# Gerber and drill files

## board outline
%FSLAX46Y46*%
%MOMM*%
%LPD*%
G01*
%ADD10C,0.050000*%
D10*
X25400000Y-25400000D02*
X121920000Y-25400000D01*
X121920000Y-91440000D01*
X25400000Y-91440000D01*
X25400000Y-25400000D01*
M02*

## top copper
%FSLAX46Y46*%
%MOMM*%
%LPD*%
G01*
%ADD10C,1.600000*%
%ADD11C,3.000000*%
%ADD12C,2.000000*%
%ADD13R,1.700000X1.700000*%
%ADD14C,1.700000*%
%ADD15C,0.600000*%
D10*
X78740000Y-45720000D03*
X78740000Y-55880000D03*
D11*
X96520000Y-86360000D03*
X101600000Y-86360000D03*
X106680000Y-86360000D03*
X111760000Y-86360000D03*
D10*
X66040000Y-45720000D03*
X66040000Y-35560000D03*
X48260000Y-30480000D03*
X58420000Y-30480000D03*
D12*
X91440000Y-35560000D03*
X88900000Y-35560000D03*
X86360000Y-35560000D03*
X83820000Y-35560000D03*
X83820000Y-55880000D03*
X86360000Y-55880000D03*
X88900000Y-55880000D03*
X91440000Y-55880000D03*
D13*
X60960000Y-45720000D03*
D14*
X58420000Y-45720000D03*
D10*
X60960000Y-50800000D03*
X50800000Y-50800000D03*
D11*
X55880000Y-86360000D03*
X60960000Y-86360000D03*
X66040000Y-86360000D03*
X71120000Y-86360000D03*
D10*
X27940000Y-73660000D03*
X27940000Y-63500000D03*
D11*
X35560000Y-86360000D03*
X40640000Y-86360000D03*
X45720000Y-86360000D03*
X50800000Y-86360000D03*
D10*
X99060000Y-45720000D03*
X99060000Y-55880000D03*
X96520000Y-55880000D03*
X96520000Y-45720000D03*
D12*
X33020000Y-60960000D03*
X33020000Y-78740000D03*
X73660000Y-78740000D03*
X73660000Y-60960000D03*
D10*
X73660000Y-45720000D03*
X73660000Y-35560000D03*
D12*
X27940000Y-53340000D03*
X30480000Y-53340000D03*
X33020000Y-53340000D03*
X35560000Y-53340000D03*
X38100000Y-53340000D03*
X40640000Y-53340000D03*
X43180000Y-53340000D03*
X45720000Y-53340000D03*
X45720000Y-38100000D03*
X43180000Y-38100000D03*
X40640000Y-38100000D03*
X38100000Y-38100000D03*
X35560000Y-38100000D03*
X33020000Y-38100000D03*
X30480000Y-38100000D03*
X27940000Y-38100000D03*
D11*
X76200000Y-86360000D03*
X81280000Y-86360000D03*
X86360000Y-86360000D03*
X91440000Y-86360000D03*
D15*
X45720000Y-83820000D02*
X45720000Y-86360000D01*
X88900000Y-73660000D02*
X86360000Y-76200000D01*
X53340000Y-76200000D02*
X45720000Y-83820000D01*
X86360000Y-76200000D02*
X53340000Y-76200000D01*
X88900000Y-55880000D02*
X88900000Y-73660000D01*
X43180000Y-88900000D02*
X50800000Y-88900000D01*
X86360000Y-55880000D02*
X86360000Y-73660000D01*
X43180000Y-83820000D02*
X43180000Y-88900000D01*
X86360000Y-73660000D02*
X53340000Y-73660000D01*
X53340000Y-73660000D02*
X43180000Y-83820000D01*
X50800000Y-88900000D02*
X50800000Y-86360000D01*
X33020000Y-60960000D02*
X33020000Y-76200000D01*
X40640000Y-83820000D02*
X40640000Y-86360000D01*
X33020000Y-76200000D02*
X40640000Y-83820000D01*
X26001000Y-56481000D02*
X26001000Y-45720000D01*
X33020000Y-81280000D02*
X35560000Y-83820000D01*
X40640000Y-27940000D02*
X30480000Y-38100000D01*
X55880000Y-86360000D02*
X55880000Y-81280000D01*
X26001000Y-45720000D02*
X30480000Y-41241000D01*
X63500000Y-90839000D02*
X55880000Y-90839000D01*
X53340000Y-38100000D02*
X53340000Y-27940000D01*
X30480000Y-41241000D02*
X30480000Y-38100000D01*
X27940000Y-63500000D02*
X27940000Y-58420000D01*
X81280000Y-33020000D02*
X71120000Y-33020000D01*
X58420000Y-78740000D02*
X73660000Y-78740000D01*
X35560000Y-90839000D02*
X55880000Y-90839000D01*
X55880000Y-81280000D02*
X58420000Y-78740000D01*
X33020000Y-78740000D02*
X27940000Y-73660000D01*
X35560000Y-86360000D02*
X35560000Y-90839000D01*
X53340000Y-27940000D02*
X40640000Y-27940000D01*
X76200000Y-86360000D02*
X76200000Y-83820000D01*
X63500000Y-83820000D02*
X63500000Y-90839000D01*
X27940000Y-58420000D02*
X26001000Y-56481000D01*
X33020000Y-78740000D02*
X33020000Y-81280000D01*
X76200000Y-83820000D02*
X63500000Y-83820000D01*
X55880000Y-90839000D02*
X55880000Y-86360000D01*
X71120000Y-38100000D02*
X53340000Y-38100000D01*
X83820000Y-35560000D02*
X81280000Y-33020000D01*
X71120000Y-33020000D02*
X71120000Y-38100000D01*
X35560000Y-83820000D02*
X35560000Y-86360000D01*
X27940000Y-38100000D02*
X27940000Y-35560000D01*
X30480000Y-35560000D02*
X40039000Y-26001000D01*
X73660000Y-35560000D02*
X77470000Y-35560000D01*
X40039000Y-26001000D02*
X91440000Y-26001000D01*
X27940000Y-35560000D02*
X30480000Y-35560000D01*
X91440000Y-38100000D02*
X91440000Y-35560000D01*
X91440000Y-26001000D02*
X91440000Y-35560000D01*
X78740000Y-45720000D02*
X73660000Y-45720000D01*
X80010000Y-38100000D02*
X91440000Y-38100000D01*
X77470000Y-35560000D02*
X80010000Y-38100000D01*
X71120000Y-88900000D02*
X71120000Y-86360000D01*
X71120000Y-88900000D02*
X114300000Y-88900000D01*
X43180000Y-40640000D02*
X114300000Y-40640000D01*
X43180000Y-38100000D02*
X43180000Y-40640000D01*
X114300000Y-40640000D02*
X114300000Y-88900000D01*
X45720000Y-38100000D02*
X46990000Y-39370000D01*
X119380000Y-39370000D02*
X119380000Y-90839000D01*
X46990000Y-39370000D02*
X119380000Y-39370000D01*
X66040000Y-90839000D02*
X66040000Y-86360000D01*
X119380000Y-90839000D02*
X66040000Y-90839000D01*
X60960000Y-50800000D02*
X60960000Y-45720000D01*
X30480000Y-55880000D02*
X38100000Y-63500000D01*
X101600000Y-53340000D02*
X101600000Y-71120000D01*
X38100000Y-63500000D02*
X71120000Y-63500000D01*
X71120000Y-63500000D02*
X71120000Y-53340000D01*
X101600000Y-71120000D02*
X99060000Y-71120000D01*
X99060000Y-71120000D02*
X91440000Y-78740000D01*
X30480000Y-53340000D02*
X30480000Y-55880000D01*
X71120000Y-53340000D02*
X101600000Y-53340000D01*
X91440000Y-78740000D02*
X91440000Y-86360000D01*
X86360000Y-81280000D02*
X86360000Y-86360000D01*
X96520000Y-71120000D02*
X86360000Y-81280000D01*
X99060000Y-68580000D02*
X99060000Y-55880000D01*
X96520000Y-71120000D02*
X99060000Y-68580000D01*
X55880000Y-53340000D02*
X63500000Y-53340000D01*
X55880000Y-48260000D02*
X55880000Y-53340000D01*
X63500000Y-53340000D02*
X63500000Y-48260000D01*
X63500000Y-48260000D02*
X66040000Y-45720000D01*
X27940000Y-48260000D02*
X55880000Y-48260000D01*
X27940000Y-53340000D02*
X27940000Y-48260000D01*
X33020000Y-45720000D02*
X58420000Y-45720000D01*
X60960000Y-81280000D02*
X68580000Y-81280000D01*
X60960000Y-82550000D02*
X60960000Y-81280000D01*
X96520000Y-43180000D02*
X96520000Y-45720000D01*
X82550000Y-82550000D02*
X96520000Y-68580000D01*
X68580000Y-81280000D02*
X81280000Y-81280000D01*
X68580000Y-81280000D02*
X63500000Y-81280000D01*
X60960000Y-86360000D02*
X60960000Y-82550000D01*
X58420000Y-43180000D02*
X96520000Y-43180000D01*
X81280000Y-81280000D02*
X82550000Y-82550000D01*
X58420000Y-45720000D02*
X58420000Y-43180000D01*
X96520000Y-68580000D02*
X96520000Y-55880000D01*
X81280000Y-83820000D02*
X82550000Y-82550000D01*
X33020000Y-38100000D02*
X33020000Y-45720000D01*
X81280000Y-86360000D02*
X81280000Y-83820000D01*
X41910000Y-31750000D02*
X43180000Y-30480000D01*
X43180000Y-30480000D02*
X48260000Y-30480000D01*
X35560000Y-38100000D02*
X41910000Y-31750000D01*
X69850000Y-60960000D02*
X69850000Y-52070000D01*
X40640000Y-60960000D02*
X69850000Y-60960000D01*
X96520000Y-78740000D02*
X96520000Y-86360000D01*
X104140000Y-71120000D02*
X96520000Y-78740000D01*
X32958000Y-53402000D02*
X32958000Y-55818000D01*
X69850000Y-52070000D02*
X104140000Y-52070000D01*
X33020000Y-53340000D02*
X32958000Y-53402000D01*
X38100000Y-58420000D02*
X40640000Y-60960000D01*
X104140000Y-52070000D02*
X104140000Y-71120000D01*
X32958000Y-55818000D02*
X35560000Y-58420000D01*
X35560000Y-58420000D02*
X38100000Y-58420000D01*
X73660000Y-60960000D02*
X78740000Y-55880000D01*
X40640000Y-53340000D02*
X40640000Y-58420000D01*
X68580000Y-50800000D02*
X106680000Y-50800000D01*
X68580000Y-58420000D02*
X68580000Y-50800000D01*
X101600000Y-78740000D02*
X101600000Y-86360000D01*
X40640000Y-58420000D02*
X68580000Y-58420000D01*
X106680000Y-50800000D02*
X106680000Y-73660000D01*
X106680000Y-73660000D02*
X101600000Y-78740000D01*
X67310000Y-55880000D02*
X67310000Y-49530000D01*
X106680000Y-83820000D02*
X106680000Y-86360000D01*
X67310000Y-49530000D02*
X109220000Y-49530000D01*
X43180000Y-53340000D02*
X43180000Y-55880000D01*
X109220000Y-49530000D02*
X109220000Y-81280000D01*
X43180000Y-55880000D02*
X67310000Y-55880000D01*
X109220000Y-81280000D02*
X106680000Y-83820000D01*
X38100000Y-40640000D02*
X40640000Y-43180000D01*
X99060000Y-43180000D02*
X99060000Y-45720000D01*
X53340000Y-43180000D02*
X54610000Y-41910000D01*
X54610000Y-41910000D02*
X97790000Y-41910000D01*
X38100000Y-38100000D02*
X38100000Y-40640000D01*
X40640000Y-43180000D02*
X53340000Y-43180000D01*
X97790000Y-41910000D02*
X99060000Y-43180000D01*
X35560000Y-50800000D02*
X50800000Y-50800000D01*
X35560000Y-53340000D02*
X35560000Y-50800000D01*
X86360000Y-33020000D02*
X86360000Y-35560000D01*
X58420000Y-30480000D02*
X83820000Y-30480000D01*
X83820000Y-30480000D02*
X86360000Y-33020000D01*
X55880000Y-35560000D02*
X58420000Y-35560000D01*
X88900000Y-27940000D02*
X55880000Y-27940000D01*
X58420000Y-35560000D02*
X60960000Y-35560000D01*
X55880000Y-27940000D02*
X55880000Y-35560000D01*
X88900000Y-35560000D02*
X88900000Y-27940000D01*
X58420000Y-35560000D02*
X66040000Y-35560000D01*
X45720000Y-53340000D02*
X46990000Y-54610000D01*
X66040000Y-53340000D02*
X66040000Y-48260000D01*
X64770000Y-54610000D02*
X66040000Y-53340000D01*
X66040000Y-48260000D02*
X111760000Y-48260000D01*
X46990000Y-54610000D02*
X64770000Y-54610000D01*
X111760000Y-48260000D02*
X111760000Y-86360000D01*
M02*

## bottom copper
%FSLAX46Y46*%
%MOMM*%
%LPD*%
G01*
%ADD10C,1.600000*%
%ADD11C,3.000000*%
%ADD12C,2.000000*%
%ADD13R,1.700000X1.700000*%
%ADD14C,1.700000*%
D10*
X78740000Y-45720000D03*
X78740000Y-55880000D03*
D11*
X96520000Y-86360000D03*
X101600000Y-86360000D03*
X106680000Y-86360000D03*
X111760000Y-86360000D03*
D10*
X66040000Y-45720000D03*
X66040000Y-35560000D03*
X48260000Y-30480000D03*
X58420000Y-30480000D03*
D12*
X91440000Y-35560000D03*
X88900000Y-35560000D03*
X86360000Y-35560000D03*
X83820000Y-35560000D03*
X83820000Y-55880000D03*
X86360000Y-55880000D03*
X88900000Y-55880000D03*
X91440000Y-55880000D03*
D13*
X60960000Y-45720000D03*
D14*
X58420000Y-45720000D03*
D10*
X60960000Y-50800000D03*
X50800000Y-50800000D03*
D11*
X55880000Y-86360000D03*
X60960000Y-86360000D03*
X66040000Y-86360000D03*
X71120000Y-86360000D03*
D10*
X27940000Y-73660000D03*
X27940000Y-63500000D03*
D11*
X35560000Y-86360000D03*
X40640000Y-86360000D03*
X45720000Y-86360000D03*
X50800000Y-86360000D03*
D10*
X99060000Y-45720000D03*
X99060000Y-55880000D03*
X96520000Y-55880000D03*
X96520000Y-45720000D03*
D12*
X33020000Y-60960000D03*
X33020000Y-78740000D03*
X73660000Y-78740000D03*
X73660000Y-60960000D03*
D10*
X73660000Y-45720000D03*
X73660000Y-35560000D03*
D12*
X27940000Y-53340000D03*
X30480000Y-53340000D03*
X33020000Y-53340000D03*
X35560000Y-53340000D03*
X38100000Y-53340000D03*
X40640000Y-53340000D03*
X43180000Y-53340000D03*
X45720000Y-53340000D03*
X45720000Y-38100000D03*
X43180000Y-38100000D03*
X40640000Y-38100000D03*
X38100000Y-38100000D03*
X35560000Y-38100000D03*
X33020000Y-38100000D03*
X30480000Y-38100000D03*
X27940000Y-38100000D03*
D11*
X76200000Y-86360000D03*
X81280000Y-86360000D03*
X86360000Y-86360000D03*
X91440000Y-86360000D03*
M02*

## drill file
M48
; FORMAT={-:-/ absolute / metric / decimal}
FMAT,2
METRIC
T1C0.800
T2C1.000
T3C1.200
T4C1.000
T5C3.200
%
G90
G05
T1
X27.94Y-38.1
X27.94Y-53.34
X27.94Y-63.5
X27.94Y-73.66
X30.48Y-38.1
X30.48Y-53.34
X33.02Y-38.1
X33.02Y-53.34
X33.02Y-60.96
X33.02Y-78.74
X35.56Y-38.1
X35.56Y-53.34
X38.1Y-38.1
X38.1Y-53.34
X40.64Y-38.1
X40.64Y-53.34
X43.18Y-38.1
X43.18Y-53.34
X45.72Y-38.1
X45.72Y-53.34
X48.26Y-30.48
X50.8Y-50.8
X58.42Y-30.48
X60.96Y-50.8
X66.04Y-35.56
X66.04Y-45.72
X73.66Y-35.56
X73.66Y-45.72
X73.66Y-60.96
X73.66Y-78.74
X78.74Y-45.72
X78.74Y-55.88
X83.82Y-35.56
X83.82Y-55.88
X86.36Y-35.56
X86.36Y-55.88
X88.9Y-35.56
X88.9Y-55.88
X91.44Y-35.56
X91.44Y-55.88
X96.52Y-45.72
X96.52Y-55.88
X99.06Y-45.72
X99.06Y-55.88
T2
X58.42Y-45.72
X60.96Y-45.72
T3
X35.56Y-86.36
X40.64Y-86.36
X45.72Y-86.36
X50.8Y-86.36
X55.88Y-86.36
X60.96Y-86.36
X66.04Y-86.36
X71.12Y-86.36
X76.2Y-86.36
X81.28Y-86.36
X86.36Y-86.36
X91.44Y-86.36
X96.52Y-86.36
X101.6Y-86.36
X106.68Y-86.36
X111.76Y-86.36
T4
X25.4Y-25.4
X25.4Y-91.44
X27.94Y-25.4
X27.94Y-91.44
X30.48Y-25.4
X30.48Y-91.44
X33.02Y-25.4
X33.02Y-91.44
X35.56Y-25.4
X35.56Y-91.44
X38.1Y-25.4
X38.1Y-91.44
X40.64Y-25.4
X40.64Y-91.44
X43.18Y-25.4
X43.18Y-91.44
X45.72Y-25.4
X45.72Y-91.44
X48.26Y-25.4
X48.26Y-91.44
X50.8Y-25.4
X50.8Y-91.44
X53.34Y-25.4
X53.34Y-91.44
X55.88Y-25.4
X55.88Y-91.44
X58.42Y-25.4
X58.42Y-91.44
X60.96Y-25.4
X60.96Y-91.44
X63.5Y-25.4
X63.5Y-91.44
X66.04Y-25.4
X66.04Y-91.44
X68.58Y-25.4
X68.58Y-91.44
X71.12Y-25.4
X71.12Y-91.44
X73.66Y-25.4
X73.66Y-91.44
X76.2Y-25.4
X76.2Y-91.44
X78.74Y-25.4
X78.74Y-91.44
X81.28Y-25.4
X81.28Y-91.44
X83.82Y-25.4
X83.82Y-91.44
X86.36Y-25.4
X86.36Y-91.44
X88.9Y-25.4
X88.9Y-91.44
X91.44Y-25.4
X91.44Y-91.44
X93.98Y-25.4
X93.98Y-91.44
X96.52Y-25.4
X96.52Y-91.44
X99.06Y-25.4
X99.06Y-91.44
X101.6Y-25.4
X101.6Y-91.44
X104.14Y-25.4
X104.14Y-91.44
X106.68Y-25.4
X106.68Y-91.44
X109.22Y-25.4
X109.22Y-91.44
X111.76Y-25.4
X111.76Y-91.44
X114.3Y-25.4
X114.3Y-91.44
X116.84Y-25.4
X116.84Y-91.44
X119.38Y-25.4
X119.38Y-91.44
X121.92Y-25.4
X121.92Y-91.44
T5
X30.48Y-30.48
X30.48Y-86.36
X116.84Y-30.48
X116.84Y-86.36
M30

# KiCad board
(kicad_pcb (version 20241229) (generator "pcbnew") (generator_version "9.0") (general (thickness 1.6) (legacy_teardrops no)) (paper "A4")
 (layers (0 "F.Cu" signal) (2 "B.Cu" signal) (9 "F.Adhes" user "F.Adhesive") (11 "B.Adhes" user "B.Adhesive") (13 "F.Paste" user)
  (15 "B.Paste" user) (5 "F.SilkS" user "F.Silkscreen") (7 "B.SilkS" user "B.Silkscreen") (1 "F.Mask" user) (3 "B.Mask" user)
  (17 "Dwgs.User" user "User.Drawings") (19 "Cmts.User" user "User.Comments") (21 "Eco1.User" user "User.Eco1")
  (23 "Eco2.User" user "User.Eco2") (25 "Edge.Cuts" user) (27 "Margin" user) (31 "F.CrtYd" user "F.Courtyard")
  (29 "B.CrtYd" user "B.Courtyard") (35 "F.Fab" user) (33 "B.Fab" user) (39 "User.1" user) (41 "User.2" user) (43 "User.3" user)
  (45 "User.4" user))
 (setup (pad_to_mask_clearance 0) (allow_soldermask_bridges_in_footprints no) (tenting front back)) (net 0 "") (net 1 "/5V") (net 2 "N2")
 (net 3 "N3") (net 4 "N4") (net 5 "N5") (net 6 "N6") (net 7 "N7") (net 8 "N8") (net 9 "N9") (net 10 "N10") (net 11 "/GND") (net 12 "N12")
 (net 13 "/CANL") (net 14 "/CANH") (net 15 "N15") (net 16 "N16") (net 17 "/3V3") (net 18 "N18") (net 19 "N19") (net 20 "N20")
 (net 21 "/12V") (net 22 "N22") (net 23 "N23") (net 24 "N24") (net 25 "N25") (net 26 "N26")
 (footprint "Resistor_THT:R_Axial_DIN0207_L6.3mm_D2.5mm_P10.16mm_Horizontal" (layer "F.Cu") (at 78.74 45.72 -90)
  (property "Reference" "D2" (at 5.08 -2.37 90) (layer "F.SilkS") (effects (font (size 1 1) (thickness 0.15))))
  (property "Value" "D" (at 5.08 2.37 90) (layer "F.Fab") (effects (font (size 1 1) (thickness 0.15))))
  (pad "1" thru_hole circle (at 0 0 270) (size 1.6 1.6) (drill 0.8) (layers "*.Cu" "*.Mask") (remove_unused_layers no) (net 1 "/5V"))
  (pad "2" thru_hole circle (at 10.16 0 270) (size 1.6 1.6) (drill 0.8) (layers "*.Cu" "*.Mask") (remove_unused_layers no) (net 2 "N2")))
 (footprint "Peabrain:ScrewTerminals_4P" (layer "F.Cu") (at 96.52 86.36 90)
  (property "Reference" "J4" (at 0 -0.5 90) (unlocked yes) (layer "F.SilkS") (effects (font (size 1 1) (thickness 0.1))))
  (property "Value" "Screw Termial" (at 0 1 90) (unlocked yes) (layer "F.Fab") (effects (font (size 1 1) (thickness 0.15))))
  (pad "1" thru_hole circle (at 0 0 90) (size 3 3) (drill 1.2) (layers "*.Cu" "F.Mask" "F.Paste") (remove_unused_layers no) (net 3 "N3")
   (thermal_bridge_angle 90))
  (pad "2" thru_hole circle (at 0 5.08 90) (size 3 3) (drill 1.2) (layers "*.Cu" "F.Mask" "F.Paste") (remove_unused_layers no) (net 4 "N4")
   (thermal_bridge_angle 90))
  (pad "3" thru_hole circle (at 0 10.16 90) (size 3 3) (drill 1.2) (layers "*.Cu" "F.Mask" "F.Paste") (remove_unused_layers no) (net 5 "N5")
   (thermal_bridge_angle 90))
  (pad "4" thru_hole circle (at 0 15.24 90) (size 3 3) (drill 1.2) (layers "*.Cu" "F.Mask" "F.Paste") (remove_unused_layers no) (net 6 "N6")
   (thermal_bridge_angle 90)))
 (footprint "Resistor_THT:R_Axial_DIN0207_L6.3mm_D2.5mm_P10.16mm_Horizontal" (layer "F.Cu") (at 66.04 45.72 90)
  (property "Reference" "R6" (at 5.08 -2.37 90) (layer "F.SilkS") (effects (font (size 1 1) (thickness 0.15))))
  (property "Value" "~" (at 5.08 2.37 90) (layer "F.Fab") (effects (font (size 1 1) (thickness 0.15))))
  (pad "1" thru_hole circle (at 0 0 90) (size 1.6 1.6) (drill 0.8) (layers "*.Cu" "*.Mask") (remove_unused_layers no) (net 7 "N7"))
  (pad "2" thru_hole circle (at 10.16 0 90) (size 1.6 1.6) (drill 0.8) (layers "*.Cu" "*.Mask") (remove_unused_layers no) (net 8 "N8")))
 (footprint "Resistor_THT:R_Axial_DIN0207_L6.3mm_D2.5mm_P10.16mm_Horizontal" (layer "F.Cu") (at 48.26 30.48)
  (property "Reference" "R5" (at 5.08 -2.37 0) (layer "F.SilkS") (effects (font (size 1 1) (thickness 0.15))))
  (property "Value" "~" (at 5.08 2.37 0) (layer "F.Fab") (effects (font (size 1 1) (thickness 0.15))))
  (pad "1" thru_hole circle (at 0 0) (size 1.6 1.6) (drill 0.8) (layers "*.Cu" "*.Mask") (remove_unused_layers no) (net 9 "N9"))
  (pad "2" thru_hole circle (at 10.16 0) (size 1.6 1.6) (drill 0.8) (layers "*.Cu" "*.Mask") (remove_unused_layers no) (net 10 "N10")))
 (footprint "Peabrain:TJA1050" (layer "F.Cu") (at 91.44 35.56 -90)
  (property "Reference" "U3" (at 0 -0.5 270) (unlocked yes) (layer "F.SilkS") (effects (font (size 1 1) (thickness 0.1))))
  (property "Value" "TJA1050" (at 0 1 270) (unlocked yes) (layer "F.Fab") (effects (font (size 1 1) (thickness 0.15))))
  (pad "1" thru_hole circle (at 0 0 270) (size 2 2) (drill 0.8) (layers "*.Cu" "F.Mask" "F.Paste") (remove_unused_layers no) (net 1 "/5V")
   (thermal_bridge_angle 90))
  (pad "2" thru_hole circle (at 0 2.54 270) (size 2 2) (drill 0.8) (layers "*.Cu" "F.Mask" "F.Paste") (remove_unused_layers no) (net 8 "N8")
   (thermal_bridge_angle 90))
  (pad "3" thru_hole circle (at 0 5.08 270) (size 2 2) (drill 0.8) (layers "*.Cu" "F.Mask" "F.Paste") (remove_unused_layers no)
   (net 10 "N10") (thermal_bridge_angle 90))
  (pad "4" thru_hole circle (at 0 7.62 270) (size 2 2) (drill 0.8) (layers "*.Cu" "F.Mask" "F.Paste") (remove_unused_layers no)
   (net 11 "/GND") (thermal_bridge_angle 90))
  (pad "5" thru_hole circle (at 20.32 7.62 270) (size 2 2) (drill 0.8) (layers "*.Cu" "F.Mask" "F.Paste") (remove_unused_layers no)
   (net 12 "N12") (thermal_bridge_angle 90))
  (pad "6" thru_hole circle (at 20.32 5.08 270) (size 2 2) (drill 0.8) (layers "*.Cu" "F.Mask" "F.Paste") (remove_unused_layers no)
   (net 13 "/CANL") (thermal_bridge_angle 90))
  (pad "7" thru_hole circle (at 20.32 2.54 270) (size 2 2) (drill 0.8) (layers "*.Cu" "F.Mask" "F.Paste") (remove_unused_layers no)
   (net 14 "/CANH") (thermal_bridge_angle 90))
  (pad "8" thru_hole circle (at 20.32 0 270) (size 2 2) (drill 0.8) (layers "*.Cu" "F.Mask" "F.Paste") (remove_unused_layers no)
   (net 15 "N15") (thermal_bridge_angle 90)))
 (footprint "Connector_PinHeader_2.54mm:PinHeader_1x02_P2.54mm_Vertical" (layer "F.Cu") (at 60.96 45.72 -90)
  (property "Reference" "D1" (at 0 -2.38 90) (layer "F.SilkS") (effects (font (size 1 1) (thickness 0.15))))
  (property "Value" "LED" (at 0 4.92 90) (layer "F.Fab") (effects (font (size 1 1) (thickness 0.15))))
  (pad "1" thru_hole rect (at 0 0 270) (size 1.7 1.7) (drill 1) (layers "*.Cu" "*.Mask") (remove_unused_layers no) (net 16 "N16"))
  (pad "2" thru_hole circle (at 0 2.54 270) (size 1.7 1.7) (drill 1) (layers "*.Cu" "*.Mask") (remove_unused_layers no) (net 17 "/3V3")))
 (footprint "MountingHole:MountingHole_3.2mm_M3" (layer "F.Cu") (at 30.48 30.48)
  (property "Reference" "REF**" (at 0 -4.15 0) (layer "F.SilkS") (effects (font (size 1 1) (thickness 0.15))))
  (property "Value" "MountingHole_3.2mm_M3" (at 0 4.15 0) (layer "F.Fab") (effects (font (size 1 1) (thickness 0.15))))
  (pad "" np_thru_hole circle (at 0 0) (size 3.2 3.2) (drill 3.2) (layers "*.Cu" "*.Mask")))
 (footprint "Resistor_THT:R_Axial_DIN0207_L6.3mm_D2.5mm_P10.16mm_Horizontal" (layer "F.Cu") (at 60.96 50.8 180)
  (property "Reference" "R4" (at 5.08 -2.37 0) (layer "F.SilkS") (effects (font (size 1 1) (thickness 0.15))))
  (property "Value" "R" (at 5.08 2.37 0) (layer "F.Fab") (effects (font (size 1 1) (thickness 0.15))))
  (pad "1" thru_hole circle (at 0 0 180) (size 1.6 1.6) (drill 0.8) (layers "*.Cu" "*.Mask") (remove_unused_layers no) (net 16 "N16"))
  (pad "2" thru_hole circle (at 10.16 0 180) (size 1.6 1.6) (drill 0.8) (layers "*.Cu" "*.Mask") (remove_unused_layers no) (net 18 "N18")))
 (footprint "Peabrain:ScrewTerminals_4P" (layer "F.Cu") (at 55.88 86.36 90)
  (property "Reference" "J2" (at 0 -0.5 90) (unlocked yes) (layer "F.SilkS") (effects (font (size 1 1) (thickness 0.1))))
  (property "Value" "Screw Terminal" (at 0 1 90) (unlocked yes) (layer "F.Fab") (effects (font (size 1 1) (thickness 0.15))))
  (pad "1" thru_hole circle (at 0 0 90) (size 3 3) (drill 1.2) (layers "*.Cu" "F.Mask" "F.Paste") (remove_unused_layers no) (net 11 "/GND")
   (thermal_bridge_angle 90))
  (pad "2" thru_hole circle (at 0 5.08 90) (size 3 3) (drill 1.2) (layers "*.Cu" "F.Mask" "F.Paste") (remove_unused_layers no)
   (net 17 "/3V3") (thermal_bridge_angle 90))
  (pad "3" thru_hole circle (at 0 10.16 90) (size 3 3) (drill 1.2) (layers "*.Cu" "F.Mask" "F.Paste") (remove_unused_layers no)
   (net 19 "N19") (thermal_bridge_angle 90))
  (pad "4" thru_hole circle (at 0 15.24 90) (size 3 3) (drill 1.2) (layers "*.Cu" "F.Mask" "F.Paste") (remove_unused_layers no)
   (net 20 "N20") (thermal_bridge_angle 90)))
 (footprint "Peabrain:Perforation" (layer "F.Cu") (at 25.4 25.4)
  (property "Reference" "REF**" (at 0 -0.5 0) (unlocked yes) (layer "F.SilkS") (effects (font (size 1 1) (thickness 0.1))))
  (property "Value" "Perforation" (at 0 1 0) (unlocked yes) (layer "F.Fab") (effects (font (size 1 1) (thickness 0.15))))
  (pad "" np_thru_hole circle (at 0 0) (size 1 1) (drill 1) (layers "F.Cu" "F.Mask" "F.Paste") (thermal_bridge_angle 90))
  (pad "" np_thru_hole circle (at 2.54 0) (size 1 1) (drill 1) (layers "F.Cu" "F.Mask" "F.Paste") (thermal_bridge_angle 90))
  (pad "" np_thru_hole circle (at 5.08 0) (size 1 1) (drill 1) (layers "F.Cu" "F.Mask" "F.Paste") (thermal_bridge_angle 90))
  (pad "" np_thru_hole circle (at 7.62 0) (size 1 1) (drill 1) (layers "F.Cu" "F.Mask" "F.Paste") (thermal_bridge_angle 90))
  (pad "" np_thru_hole circle (at 10.16 0) (size 1 1) (drill 1) (layers "F.Cu" "F.Mask" "F.Paste") (thermal_bridge_angle 90))
  (pad "" np_thru_hole circle (at 12.7 0) (size 1 1) (drill 1) (layers "F.Cu" "F.Mask" "F.Paste") (thermal_bridge_angle 90))
  (pad "" np_thru_hole circle (at 15.24 0) (size 1 1) (drill 1) (layers "F.Cu" "F.Mask" "F.Paste") (thermal_bridge_angle 90))
  (pad "" np_thru_hole circle (at 17.78 0) (size 1 1) (drill 1) (layers "F.Cu" "F.Mask" "F.Paste") (thermal_bridge_angle 90))
  (pad "" np_thru_hole circle (at 20.32 0) (size 1 1) (drill 1) (layers "F.Cu" "F.Mask" "F.Paste") (thermal_bridge_angle 90))
  (pad "" np_thru_hole circle (at 22.86 0) (size 1 1) (drill 1) (layers "F.Cu" "F.Mask" "F.Paste") (thermal_bridge_angle 90))
  (pad "" np_thru_hole circle (at 25.4 0) (size 1 1) (drill 1) (layers "F.Cu" "F.Mask" "F.Paste") (thermal_bridge_angle 90))
  (pad "" np_thru_hole circle (at 27.94 0) (size 1 1) (drill 1) (layers "F.Cu" "F.Mask" "F.Paste") (thermal_bridge_angle 90))
  (pad "" np_thru_hole circle (at 30.48 0) (size 1 1) (drill 1) (layers "F.Cu" "F.Mask" "F.Paste") (thermal_bridge_angle 90))
  (pad "" np_thru_hole circle (at 33.02 0) (size 1 1) (drill 1) (layers "F.Cu" "F.Mask" "F.Paste") (thermal_bridge_angle 90))
  (pad "" np_thru_hole circle (at 35.56 0) (size 1 1) (drill 1) (layers "F.Cu" "F.Mask" "F.Paste") (thermal_bridge_angle 90))
  (pad "" np_thru_hole circle (at 38.1 0) (size 1 1) (drill 1) (layers "F.Cu" "F.Mask" "F.Paste") (thermal_bridge_angle 90))
  (pad "" np_thru_hole circle (at 40.64 0) (size 1 1) (drill 1) (layers "F.Cu" "F.Mask" "F.Paste") (thermal_bridge_angle 90))
  (pad "" np_thru_hole circle (at 43.18 0) (size 1 1) (drill 1) (layers "F.Cu" "F.Mask" "F.Paste") (thermal_bridge_angle 90))
  (pad "" np_thru_hole circle (at 45.72 0) (size 1 1) (drill 1) (layers "F.Cu" "F.Mask" "F.Paste") (thermal_bridge_angle 90))
  (pad "" np_thru_hole circle (at 48.26 0) (size 1 1) (drill 1) (layers "F.Cu" "F.Mask" "F.Paste") (thermal_bridge_angle 90))
  (pad "" np_thru_hole circle (at 50.8 0) (size 1 1) (drill 1) (layers "F.Cu" "F.Mask" "F.Paste") (thermal_bridge_angle 90))
  (pad "" np_thru_hole circle (at 53.34 0) (size 1 1) (drill 1) (layers "F.Cu" "F.Mask" "F.Paste") (thermal_bridge_angle 90))
  (pad "" np_thru_hole circle (at 55.88 0) (size 1 1) (drill 1) (layers "F.Cu" "F.Mask" "F.Paste") (thermal_bridge_angle 90))
  (pad "" np_thru_hole circle (at 58.42 0) (size 1 1) (drill 1) (layers "F.Cu" "F.Mask" "F.Paste") (thermal_bridge_angle 90))
  (pad "" np_thru_hole circle (at 60.96 0) (size 1 1) (drill 1) (layers "F.Cu" "F.Mask" "F.Paste") (thermal_bridge_angle 90))
  (pad "" np_thru_hole circle (at 63.5 0) (size 1 1) (drill 1) (layers "F.Cu" "F.Mask" "F.Paste") (thermal_bridge_angle 90))
  (pad "" np_thru_hole circle (at 66.04 0) (size 1 1) (drill 1) (layers "F.Cu" "F.Mask" "F.Paste") (thermal_bridge_angle 90))
  (pad "" np_thru_hole circle (at 68.58 0) (size 1 1) (drill 1) (layers "F.Cu" "F.Mask" "F.Paste") (thermal_bridge_angle 90))
  (pad "" np_thru_hole circle (at 71.12 0) (size 1 1) (drill 1) (layers "F.Cu" "F.Mask" "F.Paste") (thermal_bridge_angle 90))
  (pad "" np_thru_hole circle (at 73.66 0) (size 1 1) (drill 1) (layers "F.Cu" "F.Mask" "F.Paste") (thermal_bridge_angle 90))
  (pad "" np_thru_hole circle (at 76.2 0) (size 1 1) (drill 1) (layers "F.Cu" "F.Mask" "F.Paste") (thermal_bridge_angle 90))
  (pad "" np_thru_hole circle (at 78.74 0) (size 1 1) (drill 1) (layers "F.Cu" "F.Mask" "F.Paste") (thermal_bridge_angle 90))
  (pad "" np_thru_hole circle (at 81.28 0) (size 1 1) (drill 1) (layers "F.Cu" "F.Mask" "F.Paste") (thermal_bridge_angle 90))
  (pad "" np_thru_hole circle (at 83.82 0) (size 1 1) (drill 1) (layers "F.Cu" "F.Mask" "F.Paste") (thermal_bridge_angle 90))
  (pad "" np_thru_hole circle (at 86.36 0) (size 1 1) (drill 1) (layers "F.Cu" "F.Mask" "F.Paste") (thermal_bridge_angle 90))
  (pad "" np_thru_hole circle (at 88.9 0) (size 1 1) (drill 1) (layers "F.Cu" "F.Mask" "F.Paste") (thermal_bridge_angle 90))
  (pad "" np_thru_hole circle (at 91.44 0) (size 1 1) (drill 1) (layers "F.Cu" "F.Mask" "F.Paste") (thermal_bridge_angle 90))
  (pad "" np_thru_hole circle (at 93.98 0) (size 1 1) (drill 1) (layers "F.Cu" "F.Mask" "F.Paste") (thermal_bridge_angle 90))
  (pad "" np_thru_hole circle (at 96.52 0) (size 1 1) (drill 1) (layers "F.Cu" "F.Mask" "F.Paste") (thermal_bridge_angle 90)))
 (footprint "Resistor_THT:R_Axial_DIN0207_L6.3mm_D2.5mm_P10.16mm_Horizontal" (layer "F.Cu") (at 27.94 73.66 90)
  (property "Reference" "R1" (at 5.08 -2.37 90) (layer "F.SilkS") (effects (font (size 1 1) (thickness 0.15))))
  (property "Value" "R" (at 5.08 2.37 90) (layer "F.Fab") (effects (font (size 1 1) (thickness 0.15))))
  (pad "1" thru_hole circle (at 0 0 90) (size 1.6 1.6) (drill 0.8) (layers "*.Cu" "*.Mask") (remove_unused_layers no) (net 11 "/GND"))
  (pad "2" thru_hole circle (at 10.16 0 90) (size 1.6 1.6) (drill 0.8) (layers "*.Cu" "*.Mask") (remove_unused_layers no) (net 11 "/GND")))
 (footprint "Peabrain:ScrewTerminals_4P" (layer "F.Cu") (at 35.56 86.36 90)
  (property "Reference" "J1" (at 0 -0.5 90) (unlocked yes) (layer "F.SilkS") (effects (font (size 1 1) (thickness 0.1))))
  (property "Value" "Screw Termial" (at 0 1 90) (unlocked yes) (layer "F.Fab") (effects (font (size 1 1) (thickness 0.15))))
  (pad "1" thru_hole circle (at 0 0 90) (size 3 3) (drill 1.2) (layers "*.Cu" "F.Mask" "F.Paste") (remove_unused_layers no) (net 11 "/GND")
   (thermal_bridge_angle 90))
  (pad "2" thru_hole circle (at 0 5.08 90) (size 3 3) (drill 1.2) (layers "*.Cu" "F.Mask" "F.Paste") (remove_unused_layers no)
   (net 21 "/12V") (thermal_bridge_angle 90))
  (pad "3" thru_hole circle (at 0 10.16 90) (size 3 3) (drill 1.2) (layers "*.Cu" "F.Mask" "F.Paste") (remove_unused_layers no)
   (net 14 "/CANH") (thermal_bridge_angle 90))
  (pad "4" thru_hole circle (at 0 15.24 90) (size 3 3) (drill 1.2) (layers "*.Cu" "F.Mask" "F.Paste") (remove_unused_layers no)
   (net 13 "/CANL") (thermal_bridge_angle 90)))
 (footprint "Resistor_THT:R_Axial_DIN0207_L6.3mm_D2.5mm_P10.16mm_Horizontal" (layer "F.Cu") (at 99.06 45.72 -90)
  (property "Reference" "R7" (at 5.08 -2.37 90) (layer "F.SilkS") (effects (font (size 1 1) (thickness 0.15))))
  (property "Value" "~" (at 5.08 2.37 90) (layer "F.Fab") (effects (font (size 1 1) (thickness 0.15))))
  (pad "1" thru_hole circle (at 0 0 270) (size 1.6 1.6) (drill 0.8) (layers "*.Cu" "*.Mask") (remove_unused_layers no) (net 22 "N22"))
  (pad "2" thru_hole circle (at 10.16 0 270) (size 1.6 1.6) (drill 0.8) (layers "*.Cu" "*.Mask") (remove_unused_layers no) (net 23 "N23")))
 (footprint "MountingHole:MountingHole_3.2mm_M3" (layer "F.Cu") (at 116.84 86.36)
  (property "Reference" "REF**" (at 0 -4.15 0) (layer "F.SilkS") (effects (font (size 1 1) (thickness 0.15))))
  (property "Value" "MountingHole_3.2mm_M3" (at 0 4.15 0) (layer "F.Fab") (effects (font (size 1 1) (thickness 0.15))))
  (pad "" np_thru_hole circle (at 0 0) (size 3.2 3.2) (drill 3.2) (layers "*.Cu" "*.Mask")))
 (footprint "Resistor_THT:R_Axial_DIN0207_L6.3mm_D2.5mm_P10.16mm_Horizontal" (layer "F.Cu") (at 96.52 55.88 90)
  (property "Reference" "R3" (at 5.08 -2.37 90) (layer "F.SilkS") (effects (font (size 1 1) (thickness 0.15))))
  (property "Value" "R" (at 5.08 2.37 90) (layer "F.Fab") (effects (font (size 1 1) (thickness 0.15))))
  (pad "1" thru_hole circle (at 0 0 90) (size 1.6 1.6) (drill 0.8) (layers "*.Cu" "*.Mask") (remove_unused_layers no) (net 17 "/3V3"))
  (pad "2" thru_hole circle (at 10.16 0 90) (size 1.6 1.6) (drill 0.8) (layers "*.Cu" "*.Mask") (remove_unused_layers no) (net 17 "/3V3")))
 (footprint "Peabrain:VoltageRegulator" (layer "F.Cu") (at 33.02 60.96)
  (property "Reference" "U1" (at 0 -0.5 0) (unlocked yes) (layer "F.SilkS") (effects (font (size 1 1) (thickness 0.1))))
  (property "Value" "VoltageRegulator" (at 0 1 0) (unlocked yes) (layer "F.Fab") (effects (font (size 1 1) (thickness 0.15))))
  (pad "1" thru_hole circle (at 0 0) (size 2 2) (drill 0.8) (layers "*.Cu" "F.Mask" "F.Paste") (remove_unused_layers no) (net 21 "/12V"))
  (pad "2" thru_hole circle (at 0 17.78) (size 2 2) (drill 0.8) (layers "*.Cu" "F.Mask" "F.Paste") (remove_unused_layers no) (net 11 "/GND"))
  (pad "3" thru_hole circle (at 40.64 17.78) (size 2 2) (drill 0.8) (layers "*.Cu" "F.Mask" "F.Paste") (remove_unused_layers no)
   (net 11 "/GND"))
  (pad "4" thru_hole circle (at 40.64 0) (size 2 2) (drill 0.8) (layers "*.Cu" "F.Mask" "F.Paste") (remove_unused_layers no) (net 2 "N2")))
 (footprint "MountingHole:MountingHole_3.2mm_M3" (layer "F.Cu") (at 116.84 30.48)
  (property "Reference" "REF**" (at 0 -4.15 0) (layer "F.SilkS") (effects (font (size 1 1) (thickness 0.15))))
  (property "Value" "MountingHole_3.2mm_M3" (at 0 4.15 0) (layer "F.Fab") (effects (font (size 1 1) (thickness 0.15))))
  (pad "" np_thru_hole circle (at 0 0) (size 3.2 3.2) (drill 3.2) (layers "*.Cu" "*.Mask")))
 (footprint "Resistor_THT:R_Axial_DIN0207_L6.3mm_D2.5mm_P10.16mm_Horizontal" (layer "F.Cu") (at 73.66 45.72 90)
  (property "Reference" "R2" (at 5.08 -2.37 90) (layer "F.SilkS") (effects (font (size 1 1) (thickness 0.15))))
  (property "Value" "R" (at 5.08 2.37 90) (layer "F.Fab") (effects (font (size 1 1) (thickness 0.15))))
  (pad "1" thru_hole circle (at 0 0 90) (size 1.6 1.6) (drill 0.8) (layers "*.Cu" "*.Mask") (remove_unused_layers no) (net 1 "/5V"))
  (pad "2" thru_hole circle (at 10.16 0 90) (size 1.6 1.6) (drill 0.8) (layers "*.Cu" "*.Mask") (remove_unused_layers no) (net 1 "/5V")))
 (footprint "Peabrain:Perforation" (layer "F.Cu") (at 25.4 91.44)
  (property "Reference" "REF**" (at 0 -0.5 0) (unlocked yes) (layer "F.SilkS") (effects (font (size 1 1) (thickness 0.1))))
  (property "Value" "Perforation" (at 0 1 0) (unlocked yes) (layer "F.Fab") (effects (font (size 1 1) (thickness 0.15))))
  (pad "" np_thru_hole circle (at 0 0) (size 1 1) (drill 1) (layers "F.Cu" "F.Mask" "F.Paste") (thermal_bridge_angle 90))
  (pad "" np_thru_hole circle (at 2.54 0) (size 1 1) (drill 1) (layers "F.Cu" "F.Mask" "F.Paste") (thermal_bridge_angle 90))
  (pad "" np_thru_hole circle (at 5.08 0) (size 1 1) (drill 1) (layers "F.Cu" "F.Mask" "F.Paste") (thermal_bridge_angle 90))
  (pad "" np_thru_hole circle (at 7.62 0) (size 1 1) (drill 1) (layers "F.Cu" "F.Mask" "F.Paste") (thermal_bridge_angle 90))
  (pad "" np_thru_hole circle (at 10.16 0) (size 1 1) (drill 1) (layers "F.Cu" "F.Mask" "F.Paste") (thermal_bridge_angle 90))
  (pad "" np_thru_hole circle (at 12.7 0) (size 1 1) (drill 1) (layers "F.Cu" "F.Mask" "F.Paste") (thermal_bridge_angle 90))
  (pad "" np_thru_hole circle (at 15.24 0) (size 1 1) (drill 1) (layers "F.Cu" "F.Mask" "F.Paste") (thermal_bridge_angle 90))
  (pad "" np_thru_hole circle (at 17.78 0) (size 1 1) (drill 1) (layers "F.Cu" "F.Mask" "F.Paste") (thermal_bridge_angle 90))
  (pad "" np_thru_hole circle (at 20.32 0) (size 1 1) (drill 1) (layers "F.Cu" "F.Mask" "F.Paste") (thermal_bridge_angle 90))
  (pad "" np_thru_hole circle (at 22.86 0) (size 1 1) (drill 1) (layers "F.Cu" "F.Mask" "F.Paste") (thermal_bridge_angle 90))
  (pad "" np_thru_hole circle (at 25.4 0) (size 1 1) (drill 1) (layers "F.Cu" "F.Mask" "F.Paste") (thermal_bridge_angle 90))
  (pad "" np_thru_hole circle (at 27.94 0) (size 1 1) (drill 1) (layers "F.Cu" "F.Mask" "F.Paste") (thermal_bridge_angle 90))
  (pad "" np_thru_hole circle (at 30.48 0) (size 1 1) (drill 1) (layers "F.Cu" "F.Mask" "F.Paste") (thermal_bridge_angle 90))
  (pad "" np_thru_hole circle (at 33.02 0) (size 1 1) (drill 1) (layers "F.Cu" "F.Mask" "F.Paste") (thermal_bridge_angle 90))
  (pad "" np_thru_hole circle (at 35.56 0) (size 1 1) (drill 1) (layers "F.Cu" "F.Mask" "F.Paste") (thermal_bridge_angle 90))
  (pad "" np_thru_hole circle (at 38.1 0) (size 1 1) (drill 1) (layers "F.Cu" "F.Mask" "F.Paste") (thermal_bridge_angle 90))
  (pad "" np_thru_hole circle (at 40.64 0) (size 1 1) (drill 1) (layers "F.Cu" "F.Mask" "F.Paste") (thermal_bridge_angle 90))
  (pad "" np_thru_hole circle (at 43.18 0) (size 1 1) (drill 1) (layers "F.Cu" "F.Mask" "F.Paste") (thermal_bridge_angle 90))
  (pad "" np_thru_hole circle (at 45.72 0) (size 1 1) (drill 1) (layers "F.Cu" "F.Mask" "F.Paste") (thermal_bridge_angle 90))
  (pad "" np_thru_hole circle (at 48.26 0) (size 1 1) (drill 1) (layers "F.Cu" "F.Mask" "F.Paste") (thermal_bridge_angle 90))
  (pad "" np_thru_hole circle (at 50.8 0) (size 1 1) (drill 1) (layers "F.Cu" "F.Mask" "F.Paste") (thermal_bridge_angle 90))
  (pad "" np_thru_hole circle (at 53.34 0) (size 1 1) (drill 1) (layers "F.Cu" "F.Mask" "F.Paste") (thermal_bridge_angle 90))
  (pad "" np_thru_hole circle (at 55.88 0) (size 1 1) (drill 1) (layers "F.Cu" "F.Mask" "F.Paste") (thermal_bridge_angle 90))
  (pad "" np_thru_hole circle (at 58.42 0) (size 1 1) (drill 1) (layers "F.Cu" "F.Mask" "F.Paste") (thermal_bridge_angle 90))
  (pad "" np_thru_hole circle (at 60.96 0) (size 1 1) (drill 1) (layers "F.Cu" "F.Mask" "F.Paste") (thermal_bridge_angle 90))
  (pad "" np_thru_hole circle (at 63.5 0) (size 1 1) (drill 1) (layers "F.Cu" "F.Mask" "F.Paste") (thermal_bridge_angle 90))
  (pad "" np_thru_hole circle (at 66.04 0) (size 1 1) (drill 1) (layers "F.Cu" "F.Mask" "F.Paste") (thermal_bridge_angle 90))
  (pad "" np_thru_hole circle (at 68.58 0) (size 1 1) (drill 1) (layers "F.Cu" "F.Mask" "F.Paste") (thermal_bridge_angle 90))
  (pad "" np_thru_hole circle (at 71.12 0) (size 1 1) (drill 1) (layers "F.Cu" "F.Mask" "F.Paste") (thermal_bridge_angle 90))
  (pad "" np_thru_hole circle (at 73.66 0) (size 1 1) (drill 1) (layers "F.Cu" "F.Mask" "F.Paste") (thermal_bridge_angle 90))
  (pad "" np_thru_hole circle (at 76.2 0) (size 1 1) (drill 1) (layers "F.Cu" "F.Mask" "F.Paste") (thermal_bridge_angle 90))
  (pad "" np_thru_hole circle (at 78.74 0) (size 1 1) (drill 1) (layers "F.Cu" "F.Mask" "F.Paste") (thermal_bridge_angle 90))
  (pad "" np_thru_hole circle (at 81.28 0) (size 1 1) (drill 1) (layers "F.Cu" "F.Mask" "F.Paste") (thermal_bridge_angle 90))
  (pad "" np_thru_hole circle (at 83.82 0) (size 1 1) (drill 1) (layers "F.Cu" "F.Mask" "F.Paste") (thermal_bridge_angle 90))
  (pad "" np_thru_hole circle (at 86.36 0) (size 1 1) (drill 1) (layers "F.Cu" "F.Mask" "F.Paste") (thermal_bridge_angle 90))
  (pad "" np_thru_hole circle (at 88.9 0) (size 1 1) (drill 1) (layers "F.Cu" "F.Mask" "F.Paste") (thermal_bridge_angle 90))
  (pad "" np_thru_hole circle (at 91.44 0) (size 1 1) (drill 1) (layers "F.Cu" "F.Mask" "F.Paste") (thermal_bridge_angle 90))
  (pad "" np_thru_hole circle (at 93.98 0) (size 1 1) (drill 1) (layers "F.Cu" "F.Mask" "F.Paste") (thermal_bridge_angle 90))
  (pad "" np_thru_hole circle (at 96.52 0) (size 1 1) (drill 1) (layers "F.Cu" "F.Mask" "F.Paste") (thermal_bridge_angle 90)))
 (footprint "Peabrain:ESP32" (layer "F.Cu") (at 27.94 53.34 90)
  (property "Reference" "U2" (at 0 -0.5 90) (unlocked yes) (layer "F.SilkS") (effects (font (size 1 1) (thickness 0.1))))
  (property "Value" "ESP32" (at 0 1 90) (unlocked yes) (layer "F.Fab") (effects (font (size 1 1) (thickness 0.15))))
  (pad "1" thru_hole circle (at 0 0 90) (size 2 2) (drill 0.8) (layers "*.Cu" "F.Mask" "F.Paste") (remove_unused_layers no) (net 7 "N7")
   (thermal_bridge_angle 90))
  (pad "2" thru_hole circle (at 0 2.54 90) (size 2 2) (drill 0.8) (layers "*.Cu" "F.Mask" "F.Paste") (remove_unused_layers no)
   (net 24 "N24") (thermal_bridge_angle 90))
  (pad "3" thru_hole circle (at 0 5.08 90) (size 2 2) (drill 0.8) (layers "*.Cu" "F.Mask" "F.Paste") (remove_unused_layers no) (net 3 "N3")
   (thermal_bridge_angle 90))
  (pad "4" thru_hole circle (at 0 7.62 90) (size 2 2) (drill 0.8) (layers "*.Cu" "F.Mask" "F.Paste") (remove_unused_layers no)
   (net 18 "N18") (thermal_bridge_angle 90))
  (pad "5" thru_hole circle (at 0 10.16 90) (size 2 2) (drill 0.8) (layers "*.Cu" "F.Mask" "F.Paste") (remove_unused_layers no)
   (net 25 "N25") (thermal_bridge_angle 90))
  (pad "6" thru_hole circle (at 0 12.7 90) (size 2 2) (drill 0.8) (layers "*.Cu" "F.Mask" "F.Paste") (remove_unused_layers no) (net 4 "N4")
   (thermal_bridge_angle 90))
  (pad "7" thru_hole circle (at 0 15.24 90) (size 2 2) (drill 0.8) (layers "*.Cu" "F.Mask" "F.Paste") (remove_unused_layers no) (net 5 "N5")
   (thermal_bridge_angle 90))
  (pad "8" thru_hole circle (at 0 17.78 90) (size 2 2) (drill 0.8) (layers "*.Cu" "F.Mask" "F.Paste") (remove_unused_layers no) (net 6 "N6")
   (thermal_bridge_angle 90))
  (pad "9" thru_hole circle (at 15.24 17.78 90) (size 2 2) (drill 0.8) (layers "*.Cu" "F.Mask" "F.Paste") (remove_unused_layers no)
   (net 19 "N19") (thermal_bridge_angle 90))
  (pad "10" thru_hole circle (at 15.24 15.24 90) (size 2 2) (drill 0.8) (layers "*.Cu" "F.Mask" "F.Paste") (remove_unused_layers no)
   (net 20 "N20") (thermal_bridge_angle 90))
  (pad "11" thru_hole circle (at 15.24 12.7 90) (size 2 2) (drill 0.8) (layers "*.Cu" "F.Mask" "F.Paste") (remove_unused_layers no)
   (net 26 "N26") (thermal_bridge_angle 90))
  (pad "12" thru_hole circle (at 15.24 10.16 90) (size 2 2) (drill 0.8) (layers "*.Cu" "F.Mask" "F.Paste") (remove_unused_layers no)
   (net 22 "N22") (thermal_bridge_angle 90))
  (pad "13" thru_hole circle (at 15.24 7.62 90) (size 2 2) (drill 0.8) (layers "*.Cu" "F.Mask" "F.Paste") (remove_unused_layers no)
   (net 9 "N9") (thermal_bridge_angle 90))
  (pad "14" thru_hole circle (at 15.24 5.08 90) (size 2 2) (drill 0.8) (layers "*.Cu" "F.Mask" "F.Paste") (remove_unused_layers no)
   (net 17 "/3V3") (thermal_bridge_angle 90))
  (pad "15" thru_hole circle (at 15.24 2.54 90) (size 2 2) (drill 0.8) (layers "*.Cu" "F.Mask" "F.Paste") (remove_unused_layers no)
   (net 11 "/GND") (thermal_bridge_angle 90))
  (pad "16" thru_hole circle (at 15.24 0 90) (size 2 2) (drill 0.8) (layers "*.Cu" "F.Mask" "F.Paste") (remove_unused_layers no)
   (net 1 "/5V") (thermal_bridge_angle 90)))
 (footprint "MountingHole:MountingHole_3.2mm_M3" (layer "F.Cu") (at 30.48 86.36)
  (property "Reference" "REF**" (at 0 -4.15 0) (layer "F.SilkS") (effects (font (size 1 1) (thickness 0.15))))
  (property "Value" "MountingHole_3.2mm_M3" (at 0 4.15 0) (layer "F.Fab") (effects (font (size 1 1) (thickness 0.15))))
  (pad "" np_thru_hole circle (at 0 0) (size 3.2 3.2) (drill 3.2) (layers "*.Cu" "*.Mask")))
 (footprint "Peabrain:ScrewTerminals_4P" (layer "F.Cu") (at 76.2 86.36 90)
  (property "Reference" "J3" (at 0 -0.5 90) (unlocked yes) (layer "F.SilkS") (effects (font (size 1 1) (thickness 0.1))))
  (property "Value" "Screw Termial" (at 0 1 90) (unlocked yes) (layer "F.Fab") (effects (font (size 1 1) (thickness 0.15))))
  (pad "1" thru_hole circle (at 0 0 90) (size 3 3) (drill 1.2) (layers "*.Cu" "F.Mask" "F.Paste") (remove_unused_layers no) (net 11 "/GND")
   (thermal_bridge_angle 90))
  (pad "2" thru_hole circle (at 0 5.08 90) (size 3 3) (drill 1.2) (layers "*.Cu" "F.Mask" "F.Paste") (remove_unused_layers no)
   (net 17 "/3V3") (thermal_bridge_angle 90))
  (pad "3" thru_hole circle (at 0 10.16 90) (size 3 3) (drill 1.2) (layers "*.Cu" "F.Mask" "F.Paste") (remove_unused_layers no)
   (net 23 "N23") (thermal_bridge_angle 90))
  (pad "4" thru_hole circle (at 0 15.24 90) (size 3 3) (drill 1.2) (layers "*.Cu" "F.Mask" "F.Paste") (remove_unused_layers no)
   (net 24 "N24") (thermal_bridge_angle 90)))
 (gr_rect (start 25.4 25.4) (end 121.92 91.44) (stroke (width 0.05) (type default)) (fill no) (layer "Edge.Cuts"))
 (segment (start 45.72 83.82) (end 45.72 86.36) (width 0.6) (layer "F.Cu") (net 14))
 (segment (start 88.9 73.66) (end 86.36 76.2) (width 0.6) (layer "F.Cu") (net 14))
 (segment (start 53.34 76.2) (end 45.72 83.82) (width 0.6) (layer "F.Cu") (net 14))
 (segment (start 86.36 76.2) (end 53.34 76.2) (width 0.6) (layer "F.Cu") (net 14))
 (segment (start 88.9 55.88) (end 88.9 73.66) (width 0.6) (layer "F.Cu") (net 14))
 (segment (start 43.18 88.9) (end 50.8 88.9) (width 0.6) (layer "F.Cu") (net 13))
 (segment (start 86.36 55.88) (end 86.36 73.66) (width 0.6) (layer "F.Cu") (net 13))
 (segment (start 43.18 83.82) (end 43.18 88.9) (width 0.6) (layer "F.Cu") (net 13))
 (segment (start 86.36 73.66) (end 53.34 73.66) (width 0.6) (layer "F.Cu") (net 13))
 (segment (start 53.34 73.66) (end 43.18 83.82) (width 0.6) (layer "F.Cu") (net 13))
 (segment (start 50.8 88.9) (end 50.8 86.36) (width 0.6) (layer "F.Cu") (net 13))
 (segment (start 33.02 60.96) (end 33.02 76.2) (width 0.6) (layer "F.Cu") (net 21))
 (segment (start 40.64 83.82) (end 40.64 86.36) (width 0.6) (layer "F.Cu") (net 21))
 (segment (start 33.02 76.2) (end 40.64 83.82) (width 0.6) (layer "F.Cu") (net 21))
 (segment (start 26.001 56.481) (end 26.001 45.72) (width 0.6) (layer "F.Cu") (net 11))
 (segment (start 33.02 81.28) (end 35.56 83.82) (width 0.6) (layer "F.Cu") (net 11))
 (segment (start 40.64 27.94) (end 30.48 38.1) (width 0.6) (layer "F.Cu") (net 11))
 (segment (start 55.88 86.36) (end 55.88 81.28) (width 0.6) (layer "F.Cu") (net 11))
 (segment (start 26.001 45.72) (end 30.48 41.241) (width 0.6) (layer "F.Cu") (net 11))
 (segment (start 63.5 90.839) (end 55.88 90.839) (width 0.6) (layer "F.Cu") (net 11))
 (segment (start 53.34 38.1) (end 53.34 27.94) (width 0.6) (layer "F.Cu") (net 11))
 (segment (start 30.48 41.241) (end 30.48 38.1) (width 0.6) (layer "F.Cu") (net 11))
 (segment (start 27.94 63.5) (end 27.94 58.42) (width 0.6) (layer "F.Cu") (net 11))
 (segment (start 81.28 33.02) (end 71.12 33.02) (width 0.6) (layer "F.Cu") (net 11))
 (segment (start 58.42 78.74) (end 73.66 78.74) (width 0.6) (layer "F.Cu") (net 11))
 (segment (start 35.56 90.839) (end 55.88 90.839) (width 0.6) (layer "F.Cu") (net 11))
 (segment (start 55.88 81.28) (end 58.42 78.74) (width 0.6) (layer "F.Cu") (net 11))
 (segment (start 33.02 78.74) (end 27.94 73.66) (width 0.6) (layer "F.Cu") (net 11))
 (segment (start 35.56 86.36) (end 35.56 90.839) (width 0.6) (layer "F.Cu") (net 11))
 (segment (start 53.34 27.94) (end 40.64 27.94) (width 0.6) (layer "F.Cu") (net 11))
 (segment (start 76.2 86.36) (end 76.2 83.82) (width 0.6) (layer "F.Cu") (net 11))
 (segment (start 63.5 83.82) (end 63.5 90.839) (width 0.6) (layer "F.Cu") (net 11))
 (segment (start 27.94 58.42) (end 26.001 56.481) (width 0.6) (layer "F.Cu") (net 11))
 (segment (start 33.02 78.74) (end 33.02 81.28) (width 0.6) (layer "F.Cu") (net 11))
 (segment (start 76.2 83.82) (end 63.5 83.82) (width 0.6) (layer "F.Cu") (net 11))
 (segment (start 55.88 90.839) (end 55.88 86.36) (width 0.6) (layer "F.Cu") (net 11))
 (segment (start 71.12 38.1) (end 53.34 38.1) (width 0.6) (layer "F.Cu") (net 11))
 (segment (start 83.82 35.56) (end 81.28 33.02) (width 0.6) (layer "F.Cu") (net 11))
 (segment (start 71.12 33.02) (end 71.12 38.1) (width 0.6) (layer "F.Cu") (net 11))
 (segment (start 35.56 83.82) (end 35.56 86.36) (width 0.6) (layer "F.Cu") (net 11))
 (segment (start 27.94 38.1) (end 27.94 35.56) (width 0.6) (layer "F.Cu") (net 1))
 (segment (start 30.48 35.56) (end 40.039 26.001) (width 0.6) (layer "F.Cu") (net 1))
 (segment (start 73.66 35.56) (end 77.47 35.56) (width 0.6) (layer "F.Cu") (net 1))
 (segment (start 40.039 26.001) (end 91.44 26.001) (width 0.6) (layer "F.Cu") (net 1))
 (segment (start 27.94 35.56) (end 30.48 35.56) (width 0.6) (layer "F.Cu") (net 1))
 (segment (start 91.44 38.1) (end 91.44 35.56) (width 0.6) (layer "F.Cu") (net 1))
 (segment (start 91.44 26.001) (end 91.44 35.56) (width 0.6) (layer "F.Cu") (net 1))
 (segment (start 78.74 45.72) (end 73.66 45.72) (width 0.6) (layer "F.Cu") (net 1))
 (segment (start 80.01 38.1) (end 91.44 38.1) (width 0.6) (layer "F.Cu") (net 1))
 (segment (start 77.47 35.56) (end 80.01 38.1) (width 0.6) (layer "F.Cu") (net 1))
 (segment (start 71.12 88.9) (end 71.12 86.36) (width 0.6) (layer "F.Cu") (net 20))
 (segment (start 71.12 88.9) (end 114.3 88.9) (width 0.6) (layer "F.Cu") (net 20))
 (segment (start 43.18 40.64) (end 114.3 40.64) (width 0.6) (layer "F.Cu") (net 20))
 (segment (start 43.18 38.1) (end 43.18 40.64) (width 0.6) (layer "F.Cu") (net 20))
 (segment (start 114.3 40.64) (end 114.3 88.9) (width 0.6) (layer "F.Cu") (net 20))
 (segment (start 45.72 38.1) (end 46.99 39.37) (width 0.6) (layer "F.Cu") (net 19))
 (segment (start 119.38 39.37) (end 119.38 90.839) (width 0.6) (layer "F.Cu") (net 19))
 (segment (start 46.99 39.37) (end 119.38 39.37) (width 0.6) (layer "F.Cu") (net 19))
 (segment (start 66.04 90.839) (end 66.04 86.36) (width 0.6) (layer "F.Cu") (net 19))
 (segment (start 119.38 90.839) (end 66.04 90.839) (width 0.6) (layer "F.Cu") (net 19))
 (segment (start 60.96 50.8) (end 60.96 45.72) (width 0.6) (layer "F.Cu") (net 16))
 (segment (start 30.48 55.88) (end 38.1 63.5) (width 0.6) (layer "F.Cu") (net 24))
 (segment (start 101.6 53.34) (end 101.6 71.12) (width 0.6) (layer "F.Cu") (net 24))
 (segment (start 38.1 63.5) (end 71.12 63.5) (width 0.6) (layer "F.Cu") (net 24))
 (segment (start 71.12 63.5) (end 71.12 53.34) (width 0.6) (layer "F.Cu") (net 24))
 (segment (start 101.6 71.12) (end 99.06 71.12) (width 0.6) (layer "F.Cu") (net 24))
 (segment (start 99.06 71.12) (end 91.44 78.74) (width 0.6) (layer "F.Cu") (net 24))
 (segment (start 30.48 53.34) (end 30.48 55.88) (width 0.6) (layer "F.Cu") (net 24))
 (segment (start 71.12 53.34) (end 101.6 53.34) (width 0.6) (layer "F.Cu") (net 24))
 (segment (start 91.44 78.74) (end 91.44 86.36) (width 0.6) (layer "F.Cu") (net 24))
 (segment (start 86.36 81.28) (end 86.36 86.36) (width 0.6) (layer "F.Cu") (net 23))
 (segment (start 96.52 71.12) (end 86.36 81.28) (width 0.6) (layer "F.Cu") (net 23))
 (segment (start 99.06 68.58) (end 99.06 55.88) (width 0.6) (layer "F.Cu") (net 23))
 (segment (start 96.52 71.12) (end 99.06 68.58) (width 0.6) (layer "F.Cu") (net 23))
 (segment (start 55.88 53.34) (end 63.5 53.34) (width 0.6) (layer "F.Cu") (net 7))
 (segment (start 55.88 48.26) (end 55.88 53.34) (width 0.6) (layer "F.Cu") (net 7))
 (segment (start 63.5 53.34) (end 63.5 48.26) (width 0.6) (layer "F.Cu") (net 7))
 (segment (start 63.5 48.26) (end 66.04 45.72) (width 0.6) (layer "F.Cu") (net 7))
 (segment (start 27.94 48.26) (end 55.88 48.26) (width 0.6) (layer "F.Cu") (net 7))
 (segment (start 27.94 53.34) (end 27.94 48.26) (width 0.6) (layer "F.Cu") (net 7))
 (segment (start 33.02 45.72) (end 58.42 45.72) (width 0.6) (layer "F.Cu") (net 17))
 (segment (start 60.96 81.28) (end 68.58 81.28) (width 0.6) (layer "F.Cu") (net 17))
 (segment (start 60.96 82.55) (end 60.96 81.28) (width 0.6) (layer "F.Cu") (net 17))
 (segment (start 96.52 43.18) (end 96.52 45.72) (width 0.6) (layer "F.Cu") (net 17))
 (segment (start 82.55 82.55) (end 96.52 68.58) (width 0.6) (layer "F.Cu") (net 17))
 (segment (start 68.58 81.28) (end 81.28 81.28) (width 0.6) (layer "F.Cu") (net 17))
 (segment (start 68.58 81.28) (end 63.5 81.28) (width 0.6) (layer "F.Cu") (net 17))
 (segment (start 60.96 86.36) (end 60.96 82.55) (width 0.6) (layer "F.Cu") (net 17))
 (segment (start 58.42 43.18) (end 96.52 43.18) (width 0.6) (layer "F.Cu") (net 17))
 (segment (start 81.28 81.28) (end 82.55 82.55) (width 0.6) (layer "F.Cu") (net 17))
 (segment (start 58.42 45.72) (end 58.42 43.18) (width 0.6) (layer "F.Cu") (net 17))
 (segment (start 96.52 68.58) (end 96.52 55.88) (width 0.6) (layer "F.Cu") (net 17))
 (segment (start 81.28 83.82) (end 82.55 82.55) (width 0.6) (layer "F.Cu") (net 17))
 (segment (start 33.02 38.1) (end 33.02 45.72) (width 0.6) (layer "F.Cu") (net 17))
 (segment (start 81.28 86.36) (end 81.28 83.82) (width 0.6) (layer "F.Cu") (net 17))
 (segment (start 41.91 31.75) (end 43.18 30.48) (width 0.6) (layer "F.Cu") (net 9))
 (segment (start 43.18 30.48) (end 48.26 30.48) (width 0.6) (layer "F.Cu") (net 9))
 (segment (start 35.56 38.1) (end 41.91 31.75) (width 0.6) (layer "F.Cu") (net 9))
 (segment (start 69.85 60.96) (end 69.85 52.07) (width 0.6) (layer "F.Cu") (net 3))
 (segment (start 40.64 60.96) (end 69.85 60.96) (width 0.6) (layer "F.Cu") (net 3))
 (segment (start 96.52 78.74) (end 96.52 86.36) (width 0.6) (layer "F.Cu") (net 3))
 (segment (start 104.14 71.12) (end 96.52 78.74) (width 0.6) (layer "F.Cu") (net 3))
 (segment (start 32.958 53.402) (end 32.958 55.818) (width 0.6) (layer "F.Cu") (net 3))
 (segment (start 69.85 52.07) (end 104.14 52.07) (width 0.6) (layer "F.Cu") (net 3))
 (segment (start 33.02 53.34) (end 32.958 53.402) (width 0.6) (layer "F.Cu") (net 3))
 (segment (start 38.1 58.42) (end 40.64 60.96) (width 0.6) (layer "F.Cu") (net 3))
 (segment (start 104.14 52.07) (end 104.14 71.12) (width 0.6) (layer "F.Cu") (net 3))
 (segment (start 32.958 55.818) (end 35.56 58.42) (width 0.6) (layer "F.Cu") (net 3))
 (segment (start 35.56 58.42) (end 38.1 58.42) (width 0.6) (layer "F.Cu") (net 3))
 (segment (start 73.66 60.96) (end 78.74 55.88) (width 0.6) (layer "F.Cu") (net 2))
 (segment (start 40.64 53.34) (end 40.64 58.42) (width 0.6) (layer "F.Cu") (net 4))
 (segment (start 68.58 50.8) (end 106.68 50.8) (width 0.6) (layer "F.Cu") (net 4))
 (segment (start 68.58 58.42) (end 68.58 50.8) (width 0.6) (layer "F.Cu") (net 4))
 (segment (start 101.6 78.74) (end 101.6 86.36) (width 0.6) (layer "F.Cu") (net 4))
 (segment (start 40.64 58.42) (end 68.58 58.42) (width 0.6) (layer "F.Cu") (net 4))
 (segment (start 106.68 50.8) (end 106.68 73.66) (width 0.6) (layer "F.Cu") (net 4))
 (segment (start 106.68 73.66) (end 101.6 78.74) (width 0.6) (layer "F.Cu") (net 4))
 (segment (start 67.31 55.88) (end 67.31 49.53) (width 0.6) (layer "F.Cu") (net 5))
 (segment (start 106.68 83.82) (end 106.68 86.36) (width 0.6) (layer "F.Cu") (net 5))
 (segment (start 67.31 49.53) (end 109.22 49.53) (width 0.6) (layer "F.Cu") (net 5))
 (segment (start 43.18 53.34) (end 43.18 55.88) (width 0.6) (layer "F.Cu") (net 5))
 (segment (start 109.22 49.53) (end 109.22 81.28) (width 0.6) (layer "F.Cu") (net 5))
 (segment (start 43.18 55.88) (end 67.31 55.88) (width 0.6) (layer "F.Cu") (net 5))
 (segment (start 109.22 81.28) (end 106.68 83.82) (width 0.6) (layer "F.Cu") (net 5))
 (segment (start 38.1 40.64) (end 40.64 43.18) (width 0.6) (layer "F.Cu") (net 22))
 (segment (start 99.06 43.18) (end 99.06 45.72) (width 0.6) (layer "F.Cu") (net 22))
 (segment (start 53.34 43.18) (end 54.61 41.91) (width 0.6) (layer "F.Cu") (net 22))
 (segment (start 54.61 41.91) (end 97.79 41.91) (width 0.6) (layer "F.Cu") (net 22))
 (segment (start 38.1 38.1) (end 38.1 40.64) (width 0.6) (layer "F.Cu") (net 22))
 (segment (start 40.64 43.18) (end 53.34 43.18) (width 0.6) (layer "F.Cu") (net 22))
 (segment (start 97.79 41.91) (end 99.06 43.18) (width 0.6) (layer "F.Cu") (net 22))
 (segment (start 35.56 50.8) (end 50.8 50.8) (width 0.6) (layer "F.Cu") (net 18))
 (segment (start 35.56 53.34) (end 35.56 50.8) (width 0.6) (layer "F.Cu") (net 18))
 (segment (start 86.36 33.02) (end 86.36 35.56) (width 0.6) (layer "F.Cu") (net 10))
 (segment (start 58.42 30.48) (end 83.82 30.48) (width 0.6) (layer "F.Cu") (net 10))
 (segment (start 83.82 30.48) (end 86.36 33.02) (width 0.6) (layer "F.Cu") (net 10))
 (segment (start 55.88 35.56) (end 58.42 35.56) (width 0.6) (layer "F.Cu") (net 8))
 (segment (start 88.9 27.94) (end 55.88 27.94) (width 0.6) (layer "F.Cu") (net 8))
 (segment (start 58.42 35.56) (end 60.96 35.56) (width 0.6) (layer "F.Cu") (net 8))
 (segment (start 55.88 27.94) (end 55.88 35.56) (width 0.6) (layer "F.Cu") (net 8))
 (segment (start 88.9 35.56) (end 88.9 27.94) (width 0.6) (layer "F.Cu") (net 8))
 (segment (start 58.42 35.56) (end 66.04 35.56) (width 0.6) (layer "F.Cu") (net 8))
 (segment (start 45.72 53.34) (end 46.99 54.61) (width 0.6) (layer "F.Cu") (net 6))
 (segment (start 66.04 53.34) (end 66.04 48.26) (width 0.6) (layer "F.Cu") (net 6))
 (segment (start 64.77 54.61) (end 66.04 53.34) (width 0.6) (layer "F.Cu") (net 6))
 (segment (start 66.04 48.26) (end 111.76 48.26) (width 0.6) (layer "F.Cu") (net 6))
 (segment (start 46.99 54.61) (end 64.77 54.61) (width 0.6) (layer "F.Cu") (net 6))
 (segment (start 111.76 48.26) (end 111.76 86.36) (width 0.6) (layer "F.Cu") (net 6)))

